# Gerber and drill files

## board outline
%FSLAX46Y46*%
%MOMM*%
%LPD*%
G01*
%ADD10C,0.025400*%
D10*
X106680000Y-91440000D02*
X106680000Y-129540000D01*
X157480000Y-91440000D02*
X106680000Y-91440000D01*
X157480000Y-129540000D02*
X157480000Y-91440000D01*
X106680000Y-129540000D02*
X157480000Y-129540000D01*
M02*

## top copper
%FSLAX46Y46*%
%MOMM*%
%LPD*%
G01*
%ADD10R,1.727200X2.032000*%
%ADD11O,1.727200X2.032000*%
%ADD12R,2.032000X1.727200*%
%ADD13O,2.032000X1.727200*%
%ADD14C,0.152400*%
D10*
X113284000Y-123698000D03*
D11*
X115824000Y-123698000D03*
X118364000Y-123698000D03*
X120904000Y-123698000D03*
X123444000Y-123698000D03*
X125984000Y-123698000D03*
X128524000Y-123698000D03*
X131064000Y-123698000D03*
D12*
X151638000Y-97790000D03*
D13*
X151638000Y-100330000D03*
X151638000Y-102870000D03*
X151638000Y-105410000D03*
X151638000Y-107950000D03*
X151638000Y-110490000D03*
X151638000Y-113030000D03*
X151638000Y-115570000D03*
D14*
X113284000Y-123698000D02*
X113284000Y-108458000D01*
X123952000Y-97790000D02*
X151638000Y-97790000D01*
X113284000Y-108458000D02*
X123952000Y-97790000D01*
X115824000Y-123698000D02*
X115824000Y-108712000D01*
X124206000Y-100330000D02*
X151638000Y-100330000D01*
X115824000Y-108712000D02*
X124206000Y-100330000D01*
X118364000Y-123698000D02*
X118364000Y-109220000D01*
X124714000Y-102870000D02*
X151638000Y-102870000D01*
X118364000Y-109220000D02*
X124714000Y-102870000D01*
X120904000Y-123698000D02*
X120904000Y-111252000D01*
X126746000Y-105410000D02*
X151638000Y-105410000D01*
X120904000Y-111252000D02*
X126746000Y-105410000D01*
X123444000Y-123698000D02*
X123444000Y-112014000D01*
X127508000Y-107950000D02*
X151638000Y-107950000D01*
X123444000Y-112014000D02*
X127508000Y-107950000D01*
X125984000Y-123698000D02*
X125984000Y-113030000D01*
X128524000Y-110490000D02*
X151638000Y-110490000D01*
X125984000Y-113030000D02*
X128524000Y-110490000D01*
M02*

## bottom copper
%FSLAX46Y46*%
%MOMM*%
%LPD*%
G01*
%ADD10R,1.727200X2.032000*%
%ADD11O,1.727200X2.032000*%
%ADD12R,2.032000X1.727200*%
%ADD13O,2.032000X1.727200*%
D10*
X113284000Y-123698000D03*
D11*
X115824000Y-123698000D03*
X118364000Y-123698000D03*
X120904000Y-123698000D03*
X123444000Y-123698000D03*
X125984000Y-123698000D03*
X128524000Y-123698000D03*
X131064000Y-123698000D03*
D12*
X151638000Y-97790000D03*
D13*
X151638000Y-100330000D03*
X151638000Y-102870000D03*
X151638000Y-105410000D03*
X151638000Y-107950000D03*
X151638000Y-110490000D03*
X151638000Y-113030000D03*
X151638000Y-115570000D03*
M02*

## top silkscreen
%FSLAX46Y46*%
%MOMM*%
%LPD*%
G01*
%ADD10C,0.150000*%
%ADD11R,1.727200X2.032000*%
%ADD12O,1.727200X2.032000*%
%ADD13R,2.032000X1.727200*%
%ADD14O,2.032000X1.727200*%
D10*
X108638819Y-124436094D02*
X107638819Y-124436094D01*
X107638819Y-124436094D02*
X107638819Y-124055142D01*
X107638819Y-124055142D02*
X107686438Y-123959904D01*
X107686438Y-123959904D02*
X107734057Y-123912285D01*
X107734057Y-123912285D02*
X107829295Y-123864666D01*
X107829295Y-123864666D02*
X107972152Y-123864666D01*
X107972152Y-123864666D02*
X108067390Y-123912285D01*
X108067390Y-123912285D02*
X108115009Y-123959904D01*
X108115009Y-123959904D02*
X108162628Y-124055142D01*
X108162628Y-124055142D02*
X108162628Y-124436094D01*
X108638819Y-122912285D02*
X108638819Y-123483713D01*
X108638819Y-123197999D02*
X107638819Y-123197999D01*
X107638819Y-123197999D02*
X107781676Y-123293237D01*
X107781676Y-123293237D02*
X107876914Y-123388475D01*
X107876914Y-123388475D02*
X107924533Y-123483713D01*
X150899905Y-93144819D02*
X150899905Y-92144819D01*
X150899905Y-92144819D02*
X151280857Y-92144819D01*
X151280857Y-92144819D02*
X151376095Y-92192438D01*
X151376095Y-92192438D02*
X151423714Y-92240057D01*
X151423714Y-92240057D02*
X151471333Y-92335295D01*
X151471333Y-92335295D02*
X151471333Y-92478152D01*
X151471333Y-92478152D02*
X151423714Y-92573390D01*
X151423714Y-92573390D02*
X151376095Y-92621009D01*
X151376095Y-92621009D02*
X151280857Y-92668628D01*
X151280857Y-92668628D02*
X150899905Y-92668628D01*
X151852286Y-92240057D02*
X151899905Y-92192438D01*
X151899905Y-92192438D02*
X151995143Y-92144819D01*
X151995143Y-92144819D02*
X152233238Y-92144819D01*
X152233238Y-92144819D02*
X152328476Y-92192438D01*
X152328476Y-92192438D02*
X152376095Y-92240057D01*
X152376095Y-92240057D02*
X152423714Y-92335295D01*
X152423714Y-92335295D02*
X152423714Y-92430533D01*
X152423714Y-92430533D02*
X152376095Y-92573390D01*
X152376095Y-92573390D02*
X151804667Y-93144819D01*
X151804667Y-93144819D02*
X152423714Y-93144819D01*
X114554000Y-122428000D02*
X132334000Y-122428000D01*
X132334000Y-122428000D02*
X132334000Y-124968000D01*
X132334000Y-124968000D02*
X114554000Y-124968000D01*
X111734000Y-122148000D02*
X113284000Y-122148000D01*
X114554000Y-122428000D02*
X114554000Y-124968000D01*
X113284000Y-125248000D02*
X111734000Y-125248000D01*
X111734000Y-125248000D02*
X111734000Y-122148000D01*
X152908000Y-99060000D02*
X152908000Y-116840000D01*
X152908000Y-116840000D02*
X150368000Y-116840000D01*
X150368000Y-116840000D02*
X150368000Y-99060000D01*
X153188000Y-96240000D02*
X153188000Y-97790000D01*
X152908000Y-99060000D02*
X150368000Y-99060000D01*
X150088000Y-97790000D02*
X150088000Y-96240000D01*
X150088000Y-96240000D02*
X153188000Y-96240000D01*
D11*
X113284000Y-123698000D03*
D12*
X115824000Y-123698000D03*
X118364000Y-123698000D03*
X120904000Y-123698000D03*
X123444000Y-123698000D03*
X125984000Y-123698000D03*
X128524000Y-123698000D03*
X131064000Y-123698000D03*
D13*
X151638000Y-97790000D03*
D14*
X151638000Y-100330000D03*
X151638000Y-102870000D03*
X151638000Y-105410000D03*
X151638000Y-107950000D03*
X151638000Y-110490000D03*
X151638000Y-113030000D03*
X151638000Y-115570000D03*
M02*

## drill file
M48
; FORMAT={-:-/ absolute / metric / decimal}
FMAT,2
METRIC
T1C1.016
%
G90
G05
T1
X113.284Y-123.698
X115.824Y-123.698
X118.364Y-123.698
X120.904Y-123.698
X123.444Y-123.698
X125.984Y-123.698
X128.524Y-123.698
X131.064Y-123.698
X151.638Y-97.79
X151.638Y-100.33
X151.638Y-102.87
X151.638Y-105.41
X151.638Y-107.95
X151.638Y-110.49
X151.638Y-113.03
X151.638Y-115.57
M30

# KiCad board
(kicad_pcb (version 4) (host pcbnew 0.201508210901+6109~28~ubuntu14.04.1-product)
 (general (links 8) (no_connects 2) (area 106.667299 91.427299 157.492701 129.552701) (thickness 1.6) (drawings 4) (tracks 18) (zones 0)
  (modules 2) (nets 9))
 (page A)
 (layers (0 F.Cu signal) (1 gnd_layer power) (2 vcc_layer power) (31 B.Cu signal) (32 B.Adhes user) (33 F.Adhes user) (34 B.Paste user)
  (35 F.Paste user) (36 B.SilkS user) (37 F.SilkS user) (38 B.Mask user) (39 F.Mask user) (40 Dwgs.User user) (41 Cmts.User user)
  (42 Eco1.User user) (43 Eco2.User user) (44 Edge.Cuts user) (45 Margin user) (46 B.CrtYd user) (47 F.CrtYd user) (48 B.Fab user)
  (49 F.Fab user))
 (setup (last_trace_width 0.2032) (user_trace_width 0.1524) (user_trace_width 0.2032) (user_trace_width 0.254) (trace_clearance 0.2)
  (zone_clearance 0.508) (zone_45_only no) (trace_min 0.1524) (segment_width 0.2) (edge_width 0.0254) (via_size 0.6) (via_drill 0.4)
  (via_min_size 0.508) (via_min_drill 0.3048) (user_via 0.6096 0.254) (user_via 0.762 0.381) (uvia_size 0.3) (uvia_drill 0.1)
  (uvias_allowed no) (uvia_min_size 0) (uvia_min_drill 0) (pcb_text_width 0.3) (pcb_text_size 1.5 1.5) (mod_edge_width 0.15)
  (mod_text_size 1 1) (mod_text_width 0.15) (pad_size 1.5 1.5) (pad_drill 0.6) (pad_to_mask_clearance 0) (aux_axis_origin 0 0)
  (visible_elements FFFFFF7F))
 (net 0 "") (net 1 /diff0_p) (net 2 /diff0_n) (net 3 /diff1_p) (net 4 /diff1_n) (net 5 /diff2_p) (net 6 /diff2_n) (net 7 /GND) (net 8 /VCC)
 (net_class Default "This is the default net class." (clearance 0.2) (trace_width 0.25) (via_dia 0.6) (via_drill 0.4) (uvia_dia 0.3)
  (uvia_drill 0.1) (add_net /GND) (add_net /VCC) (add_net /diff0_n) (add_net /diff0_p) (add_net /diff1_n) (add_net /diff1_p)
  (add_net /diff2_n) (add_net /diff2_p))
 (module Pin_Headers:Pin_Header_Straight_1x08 (layer F.Cu) (at 113.284 123.698 90)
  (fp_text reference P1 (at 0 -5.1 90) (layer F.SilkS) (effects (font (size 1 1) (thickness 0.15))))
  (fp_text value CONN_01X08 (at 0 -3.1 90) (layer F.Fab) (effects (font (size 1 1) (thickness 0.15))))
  (fp_line (start 1.27 1.27) (end 1.27 19.05) (layer F.SilkS) (width 0.15))
  (fp_line (start 1.27 19.05) (end -1.27 19.05) (layer F.SilkS) (width 0.15))
  (fp_line (start -1.27 19.05) (end -1.27 1.27) (layer F.SilkS) (width 0.15))
  (fp_line (start 1.55 -1.55) (end 1.55 0) (layer F.SilkS) (width 0.15))
  (fp_line (start 1.27 1.27) (end -1.27 1.27) (layer F.SilkS) (width 0.15))
  (fp_line (start -1.55 0) (end -1.55 -1.55) (layer F.SilkS) (width 0.15))
  (fp_line (start -1.55 -1.55) (end 1.55 -1.55) (layer F.SilkS) (width 0.15))
  (pad 1 thru_hole rect (at 0 0 90) (size 2.032 1.7272) (drill 1.016) (layers *.Cu *.Mask F.SilkS) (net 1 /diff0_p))
  (pad 2 thru_hole oval (at 0 2.54 90) (size 2.032 1.7272) (drill 1.016) (layers *.Cu *.Mask F.SilkS) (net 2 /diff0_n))
  (pad 3 thru_hole oval (at 0 5.08 90) (size 2.032 1.7272) (drill 1.016) (layers *.Cu *.Mask F.SilkS) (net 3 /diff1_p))
  (pad 4 thru_hole oval (at 0 7.62 90) (size 2.032 1.7272) (drill 1.016) (layers *.Cu *.Mask F.SilkS) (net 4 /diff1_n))
  (pad 5 thru_hole oval (at 0 10.16 90) (size 2.032 1.7272) (drill 1.016) (layers *.Cu *.Mask F.SilkS) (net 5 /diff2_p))
  (pad 6 thru_hole oval (at 0 12.7 90) (size 2.032 1.7272) (drill 1.016) (layers *.Cu *.Mask F.SilkS) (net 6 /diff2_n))
  (pad 7 thru_hole oval (at 0 15.24 90) (size 2.032 1.7272) (drill 1.016) (layers *.Cu *.Mask F.SilkS) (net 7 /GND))
  (pad 8 thru_hole oval (at 0 17.78 90) (size 2.032 1.7272) (drill 1.016) (layers *.Cu *.Mask F.SilkS) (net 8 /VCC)))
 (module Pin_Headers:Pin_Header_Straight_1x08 (layer F.Cu) (at 151.638 97.79)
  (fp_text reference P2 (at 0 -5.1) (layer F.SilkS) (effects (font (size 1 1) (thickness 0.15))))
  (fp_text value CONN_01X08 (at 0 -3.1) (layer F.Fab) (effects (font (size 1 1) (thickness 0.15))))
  (fp_line (start 1.27 1.27) (end 1.27 19.05) (layer F.SilkS) (width 0.15))
  (fp_line (start 1.27 19.05) (end -1.27 19.05) (layer F.SilkS) (width 0.15))
  (fp_line (start -1.27 19.05) (end -1.27 1.27) (layer F.SilkS) (width 0.15))
  (fp_line (start 1.55 -1.55) (end 1.55 0) (layer F.SilkS) (width 0.15))
  (fp_line (start 1.27 1.27) (end -1.27 1.27) (layer F.SilkS) (width 0.15))
  (fp_line (start -1.55 0) (end -1.55 -1.55) (layer F.SilkS) (width 0.15))
  (fp_line (start -1.55 -1.55) (end 1.55 -1.55) (layer F.SilkS) (width 0.15))
  (pad 1 thru_hole rect (at 0 0) (size 2.032 1.7272) (drill 1.016) (layers *.Cu *.Mask F.SilkS) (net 1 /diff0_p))
  (pad 2 thru_hole oval (at 0 2.54) (size 2.032 1.7272) (drill 1.016) (layers *.Cu *.Mask F.SilkS) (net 2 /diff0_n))
  (pad 3 thru_hole oval (at 0 5.08) (size 2.032 1.7272) (drill 1.016) (layers *.Cu *.Mask F.SilkS) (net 3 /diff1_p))
  (pad 4 thru_hole oval (at 0 7.62) (size 2.032 1.7272) (drill 1.016) (layers *.Cu *.Mask F.SilkS) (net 4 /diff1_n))
  (pad 5 thru_hole oval (at 0 10.16) (size 2.032 1.7272) (drill 1.016) (layers *.Cu *.Mask F.SilkS) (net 5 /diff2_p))
  (pad 6 thru_hole oval (at 0 12.7) (size 2.032 1.7272) (drill 1.016) (layers *.Cu *.Mask F.SilkS) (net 6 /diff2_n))
  (pad 7 thru_hole oval (at 0 15.24) (size 2.032 1.7272) (drill 1.016) (layers *.Cu *.Mask F.SilkS) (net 7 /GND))
  (pad 8 thru_hole oval (at 0 17.78) (size 2.032 1.7272) (drill 1.016) (layers *.Cu *.Mask F.SilkS) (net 8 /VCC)))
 (gr_line (start 106.68 91.44) (end 106.68 129.54) (angle 90) (layer Edge.Cuts) (width 0.0254))
 (gr_line (start 157.48 91.44) (end 106.68 91.44) (angle 90) (layer Edge.Cuts) (width 0.0254))
 (gr_line (start 157.48 129.54) (end 157.48 91.44) (angle 90) (layer Edge.Cuts) (width 0.0254))
 (gr_line (start 106.68 129.54) (end 157.48 129.54) (angle 90) (layer Edge.Cuts) (width 0.0254))
 (segment (start 113.284 123.698) (end 113.284 108.458) (width 0.1524) (layer F.Cu) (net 1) (status 400000))
 (segment (start 123.952 97.79) (end 151.638 97.79) (width 0.1524) (layer F.Cu) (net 1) (status 800000))
 (segment (start 113.284 108.458) (end 123.952 97.79) (width 0.1524) (layer F.Cu) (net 1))
 (segment (start 115.824 123.698) (end 115.824 108.712) (width 0.1524) (layer F.Cu) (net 2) (status 400000))
 (segment (start 124.206 100.33) (end 151.638 100.33) (width 0.1524) (layer F.Cu) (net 2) (status 800000))
 (segment (start 115.824 108.712) (end 124.206 100.33) (width 0.1524) (layer F.Cu) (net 2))
 (segment (start 118.364 123.698) (end 118.364 109.22) (width 0.1524) (layer F.Cu) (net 3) (status 400000))
 (segment (start 124.714 102.87) (end 151.638 102.87) (width 0.1524) (layer F.Cu) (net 3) (status 800000))
 (segment (start 118.364 109.22) (end 124.714 102.87) (width 0.1524) (layer F.Cu) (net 3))
 (segment (start 120.904 123.698) (end 120.904 111.252) (width 0.1524) (layer F.Cu) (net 4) (status 400000))
 (segment (start 126.746 105.41) (end 151.638 105.41) (width 0.1524) (layer F.Cu) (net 4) (status 800000))
 (segment (start 120.904 111.252) (end 126.746 105.41) (width 0.1524) (layer F.Cu) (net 4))
 (segment (start 123.444 123.698) (end 123.444 112.014) (width 0.1524) (layer F.Cu) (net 5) (status 400000))
 (segment (start 127.508 107.95) (end 151.638 107.95) (width 0.1524) (layer F.Cu) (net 5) (status 800000))
 (segment (start 123.444 112.014) (end 127.508 107.95) (width 0.1524) (layer F.Cu) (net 5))
 (segment (start 125.984 123.698) (end 125.984 113.03) (width 0.1524) (layer F.Cu) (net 6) (status 400000))
 (segment (start 128.524 110.49) (end 151.638 110.49) (width 0.1524) (layer F.Cu) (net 6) (status 800000))
 (segment (start 125.984 113.03) (end 128.524 110.49) (width 0.1524) (layer F.Cu) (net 6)))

